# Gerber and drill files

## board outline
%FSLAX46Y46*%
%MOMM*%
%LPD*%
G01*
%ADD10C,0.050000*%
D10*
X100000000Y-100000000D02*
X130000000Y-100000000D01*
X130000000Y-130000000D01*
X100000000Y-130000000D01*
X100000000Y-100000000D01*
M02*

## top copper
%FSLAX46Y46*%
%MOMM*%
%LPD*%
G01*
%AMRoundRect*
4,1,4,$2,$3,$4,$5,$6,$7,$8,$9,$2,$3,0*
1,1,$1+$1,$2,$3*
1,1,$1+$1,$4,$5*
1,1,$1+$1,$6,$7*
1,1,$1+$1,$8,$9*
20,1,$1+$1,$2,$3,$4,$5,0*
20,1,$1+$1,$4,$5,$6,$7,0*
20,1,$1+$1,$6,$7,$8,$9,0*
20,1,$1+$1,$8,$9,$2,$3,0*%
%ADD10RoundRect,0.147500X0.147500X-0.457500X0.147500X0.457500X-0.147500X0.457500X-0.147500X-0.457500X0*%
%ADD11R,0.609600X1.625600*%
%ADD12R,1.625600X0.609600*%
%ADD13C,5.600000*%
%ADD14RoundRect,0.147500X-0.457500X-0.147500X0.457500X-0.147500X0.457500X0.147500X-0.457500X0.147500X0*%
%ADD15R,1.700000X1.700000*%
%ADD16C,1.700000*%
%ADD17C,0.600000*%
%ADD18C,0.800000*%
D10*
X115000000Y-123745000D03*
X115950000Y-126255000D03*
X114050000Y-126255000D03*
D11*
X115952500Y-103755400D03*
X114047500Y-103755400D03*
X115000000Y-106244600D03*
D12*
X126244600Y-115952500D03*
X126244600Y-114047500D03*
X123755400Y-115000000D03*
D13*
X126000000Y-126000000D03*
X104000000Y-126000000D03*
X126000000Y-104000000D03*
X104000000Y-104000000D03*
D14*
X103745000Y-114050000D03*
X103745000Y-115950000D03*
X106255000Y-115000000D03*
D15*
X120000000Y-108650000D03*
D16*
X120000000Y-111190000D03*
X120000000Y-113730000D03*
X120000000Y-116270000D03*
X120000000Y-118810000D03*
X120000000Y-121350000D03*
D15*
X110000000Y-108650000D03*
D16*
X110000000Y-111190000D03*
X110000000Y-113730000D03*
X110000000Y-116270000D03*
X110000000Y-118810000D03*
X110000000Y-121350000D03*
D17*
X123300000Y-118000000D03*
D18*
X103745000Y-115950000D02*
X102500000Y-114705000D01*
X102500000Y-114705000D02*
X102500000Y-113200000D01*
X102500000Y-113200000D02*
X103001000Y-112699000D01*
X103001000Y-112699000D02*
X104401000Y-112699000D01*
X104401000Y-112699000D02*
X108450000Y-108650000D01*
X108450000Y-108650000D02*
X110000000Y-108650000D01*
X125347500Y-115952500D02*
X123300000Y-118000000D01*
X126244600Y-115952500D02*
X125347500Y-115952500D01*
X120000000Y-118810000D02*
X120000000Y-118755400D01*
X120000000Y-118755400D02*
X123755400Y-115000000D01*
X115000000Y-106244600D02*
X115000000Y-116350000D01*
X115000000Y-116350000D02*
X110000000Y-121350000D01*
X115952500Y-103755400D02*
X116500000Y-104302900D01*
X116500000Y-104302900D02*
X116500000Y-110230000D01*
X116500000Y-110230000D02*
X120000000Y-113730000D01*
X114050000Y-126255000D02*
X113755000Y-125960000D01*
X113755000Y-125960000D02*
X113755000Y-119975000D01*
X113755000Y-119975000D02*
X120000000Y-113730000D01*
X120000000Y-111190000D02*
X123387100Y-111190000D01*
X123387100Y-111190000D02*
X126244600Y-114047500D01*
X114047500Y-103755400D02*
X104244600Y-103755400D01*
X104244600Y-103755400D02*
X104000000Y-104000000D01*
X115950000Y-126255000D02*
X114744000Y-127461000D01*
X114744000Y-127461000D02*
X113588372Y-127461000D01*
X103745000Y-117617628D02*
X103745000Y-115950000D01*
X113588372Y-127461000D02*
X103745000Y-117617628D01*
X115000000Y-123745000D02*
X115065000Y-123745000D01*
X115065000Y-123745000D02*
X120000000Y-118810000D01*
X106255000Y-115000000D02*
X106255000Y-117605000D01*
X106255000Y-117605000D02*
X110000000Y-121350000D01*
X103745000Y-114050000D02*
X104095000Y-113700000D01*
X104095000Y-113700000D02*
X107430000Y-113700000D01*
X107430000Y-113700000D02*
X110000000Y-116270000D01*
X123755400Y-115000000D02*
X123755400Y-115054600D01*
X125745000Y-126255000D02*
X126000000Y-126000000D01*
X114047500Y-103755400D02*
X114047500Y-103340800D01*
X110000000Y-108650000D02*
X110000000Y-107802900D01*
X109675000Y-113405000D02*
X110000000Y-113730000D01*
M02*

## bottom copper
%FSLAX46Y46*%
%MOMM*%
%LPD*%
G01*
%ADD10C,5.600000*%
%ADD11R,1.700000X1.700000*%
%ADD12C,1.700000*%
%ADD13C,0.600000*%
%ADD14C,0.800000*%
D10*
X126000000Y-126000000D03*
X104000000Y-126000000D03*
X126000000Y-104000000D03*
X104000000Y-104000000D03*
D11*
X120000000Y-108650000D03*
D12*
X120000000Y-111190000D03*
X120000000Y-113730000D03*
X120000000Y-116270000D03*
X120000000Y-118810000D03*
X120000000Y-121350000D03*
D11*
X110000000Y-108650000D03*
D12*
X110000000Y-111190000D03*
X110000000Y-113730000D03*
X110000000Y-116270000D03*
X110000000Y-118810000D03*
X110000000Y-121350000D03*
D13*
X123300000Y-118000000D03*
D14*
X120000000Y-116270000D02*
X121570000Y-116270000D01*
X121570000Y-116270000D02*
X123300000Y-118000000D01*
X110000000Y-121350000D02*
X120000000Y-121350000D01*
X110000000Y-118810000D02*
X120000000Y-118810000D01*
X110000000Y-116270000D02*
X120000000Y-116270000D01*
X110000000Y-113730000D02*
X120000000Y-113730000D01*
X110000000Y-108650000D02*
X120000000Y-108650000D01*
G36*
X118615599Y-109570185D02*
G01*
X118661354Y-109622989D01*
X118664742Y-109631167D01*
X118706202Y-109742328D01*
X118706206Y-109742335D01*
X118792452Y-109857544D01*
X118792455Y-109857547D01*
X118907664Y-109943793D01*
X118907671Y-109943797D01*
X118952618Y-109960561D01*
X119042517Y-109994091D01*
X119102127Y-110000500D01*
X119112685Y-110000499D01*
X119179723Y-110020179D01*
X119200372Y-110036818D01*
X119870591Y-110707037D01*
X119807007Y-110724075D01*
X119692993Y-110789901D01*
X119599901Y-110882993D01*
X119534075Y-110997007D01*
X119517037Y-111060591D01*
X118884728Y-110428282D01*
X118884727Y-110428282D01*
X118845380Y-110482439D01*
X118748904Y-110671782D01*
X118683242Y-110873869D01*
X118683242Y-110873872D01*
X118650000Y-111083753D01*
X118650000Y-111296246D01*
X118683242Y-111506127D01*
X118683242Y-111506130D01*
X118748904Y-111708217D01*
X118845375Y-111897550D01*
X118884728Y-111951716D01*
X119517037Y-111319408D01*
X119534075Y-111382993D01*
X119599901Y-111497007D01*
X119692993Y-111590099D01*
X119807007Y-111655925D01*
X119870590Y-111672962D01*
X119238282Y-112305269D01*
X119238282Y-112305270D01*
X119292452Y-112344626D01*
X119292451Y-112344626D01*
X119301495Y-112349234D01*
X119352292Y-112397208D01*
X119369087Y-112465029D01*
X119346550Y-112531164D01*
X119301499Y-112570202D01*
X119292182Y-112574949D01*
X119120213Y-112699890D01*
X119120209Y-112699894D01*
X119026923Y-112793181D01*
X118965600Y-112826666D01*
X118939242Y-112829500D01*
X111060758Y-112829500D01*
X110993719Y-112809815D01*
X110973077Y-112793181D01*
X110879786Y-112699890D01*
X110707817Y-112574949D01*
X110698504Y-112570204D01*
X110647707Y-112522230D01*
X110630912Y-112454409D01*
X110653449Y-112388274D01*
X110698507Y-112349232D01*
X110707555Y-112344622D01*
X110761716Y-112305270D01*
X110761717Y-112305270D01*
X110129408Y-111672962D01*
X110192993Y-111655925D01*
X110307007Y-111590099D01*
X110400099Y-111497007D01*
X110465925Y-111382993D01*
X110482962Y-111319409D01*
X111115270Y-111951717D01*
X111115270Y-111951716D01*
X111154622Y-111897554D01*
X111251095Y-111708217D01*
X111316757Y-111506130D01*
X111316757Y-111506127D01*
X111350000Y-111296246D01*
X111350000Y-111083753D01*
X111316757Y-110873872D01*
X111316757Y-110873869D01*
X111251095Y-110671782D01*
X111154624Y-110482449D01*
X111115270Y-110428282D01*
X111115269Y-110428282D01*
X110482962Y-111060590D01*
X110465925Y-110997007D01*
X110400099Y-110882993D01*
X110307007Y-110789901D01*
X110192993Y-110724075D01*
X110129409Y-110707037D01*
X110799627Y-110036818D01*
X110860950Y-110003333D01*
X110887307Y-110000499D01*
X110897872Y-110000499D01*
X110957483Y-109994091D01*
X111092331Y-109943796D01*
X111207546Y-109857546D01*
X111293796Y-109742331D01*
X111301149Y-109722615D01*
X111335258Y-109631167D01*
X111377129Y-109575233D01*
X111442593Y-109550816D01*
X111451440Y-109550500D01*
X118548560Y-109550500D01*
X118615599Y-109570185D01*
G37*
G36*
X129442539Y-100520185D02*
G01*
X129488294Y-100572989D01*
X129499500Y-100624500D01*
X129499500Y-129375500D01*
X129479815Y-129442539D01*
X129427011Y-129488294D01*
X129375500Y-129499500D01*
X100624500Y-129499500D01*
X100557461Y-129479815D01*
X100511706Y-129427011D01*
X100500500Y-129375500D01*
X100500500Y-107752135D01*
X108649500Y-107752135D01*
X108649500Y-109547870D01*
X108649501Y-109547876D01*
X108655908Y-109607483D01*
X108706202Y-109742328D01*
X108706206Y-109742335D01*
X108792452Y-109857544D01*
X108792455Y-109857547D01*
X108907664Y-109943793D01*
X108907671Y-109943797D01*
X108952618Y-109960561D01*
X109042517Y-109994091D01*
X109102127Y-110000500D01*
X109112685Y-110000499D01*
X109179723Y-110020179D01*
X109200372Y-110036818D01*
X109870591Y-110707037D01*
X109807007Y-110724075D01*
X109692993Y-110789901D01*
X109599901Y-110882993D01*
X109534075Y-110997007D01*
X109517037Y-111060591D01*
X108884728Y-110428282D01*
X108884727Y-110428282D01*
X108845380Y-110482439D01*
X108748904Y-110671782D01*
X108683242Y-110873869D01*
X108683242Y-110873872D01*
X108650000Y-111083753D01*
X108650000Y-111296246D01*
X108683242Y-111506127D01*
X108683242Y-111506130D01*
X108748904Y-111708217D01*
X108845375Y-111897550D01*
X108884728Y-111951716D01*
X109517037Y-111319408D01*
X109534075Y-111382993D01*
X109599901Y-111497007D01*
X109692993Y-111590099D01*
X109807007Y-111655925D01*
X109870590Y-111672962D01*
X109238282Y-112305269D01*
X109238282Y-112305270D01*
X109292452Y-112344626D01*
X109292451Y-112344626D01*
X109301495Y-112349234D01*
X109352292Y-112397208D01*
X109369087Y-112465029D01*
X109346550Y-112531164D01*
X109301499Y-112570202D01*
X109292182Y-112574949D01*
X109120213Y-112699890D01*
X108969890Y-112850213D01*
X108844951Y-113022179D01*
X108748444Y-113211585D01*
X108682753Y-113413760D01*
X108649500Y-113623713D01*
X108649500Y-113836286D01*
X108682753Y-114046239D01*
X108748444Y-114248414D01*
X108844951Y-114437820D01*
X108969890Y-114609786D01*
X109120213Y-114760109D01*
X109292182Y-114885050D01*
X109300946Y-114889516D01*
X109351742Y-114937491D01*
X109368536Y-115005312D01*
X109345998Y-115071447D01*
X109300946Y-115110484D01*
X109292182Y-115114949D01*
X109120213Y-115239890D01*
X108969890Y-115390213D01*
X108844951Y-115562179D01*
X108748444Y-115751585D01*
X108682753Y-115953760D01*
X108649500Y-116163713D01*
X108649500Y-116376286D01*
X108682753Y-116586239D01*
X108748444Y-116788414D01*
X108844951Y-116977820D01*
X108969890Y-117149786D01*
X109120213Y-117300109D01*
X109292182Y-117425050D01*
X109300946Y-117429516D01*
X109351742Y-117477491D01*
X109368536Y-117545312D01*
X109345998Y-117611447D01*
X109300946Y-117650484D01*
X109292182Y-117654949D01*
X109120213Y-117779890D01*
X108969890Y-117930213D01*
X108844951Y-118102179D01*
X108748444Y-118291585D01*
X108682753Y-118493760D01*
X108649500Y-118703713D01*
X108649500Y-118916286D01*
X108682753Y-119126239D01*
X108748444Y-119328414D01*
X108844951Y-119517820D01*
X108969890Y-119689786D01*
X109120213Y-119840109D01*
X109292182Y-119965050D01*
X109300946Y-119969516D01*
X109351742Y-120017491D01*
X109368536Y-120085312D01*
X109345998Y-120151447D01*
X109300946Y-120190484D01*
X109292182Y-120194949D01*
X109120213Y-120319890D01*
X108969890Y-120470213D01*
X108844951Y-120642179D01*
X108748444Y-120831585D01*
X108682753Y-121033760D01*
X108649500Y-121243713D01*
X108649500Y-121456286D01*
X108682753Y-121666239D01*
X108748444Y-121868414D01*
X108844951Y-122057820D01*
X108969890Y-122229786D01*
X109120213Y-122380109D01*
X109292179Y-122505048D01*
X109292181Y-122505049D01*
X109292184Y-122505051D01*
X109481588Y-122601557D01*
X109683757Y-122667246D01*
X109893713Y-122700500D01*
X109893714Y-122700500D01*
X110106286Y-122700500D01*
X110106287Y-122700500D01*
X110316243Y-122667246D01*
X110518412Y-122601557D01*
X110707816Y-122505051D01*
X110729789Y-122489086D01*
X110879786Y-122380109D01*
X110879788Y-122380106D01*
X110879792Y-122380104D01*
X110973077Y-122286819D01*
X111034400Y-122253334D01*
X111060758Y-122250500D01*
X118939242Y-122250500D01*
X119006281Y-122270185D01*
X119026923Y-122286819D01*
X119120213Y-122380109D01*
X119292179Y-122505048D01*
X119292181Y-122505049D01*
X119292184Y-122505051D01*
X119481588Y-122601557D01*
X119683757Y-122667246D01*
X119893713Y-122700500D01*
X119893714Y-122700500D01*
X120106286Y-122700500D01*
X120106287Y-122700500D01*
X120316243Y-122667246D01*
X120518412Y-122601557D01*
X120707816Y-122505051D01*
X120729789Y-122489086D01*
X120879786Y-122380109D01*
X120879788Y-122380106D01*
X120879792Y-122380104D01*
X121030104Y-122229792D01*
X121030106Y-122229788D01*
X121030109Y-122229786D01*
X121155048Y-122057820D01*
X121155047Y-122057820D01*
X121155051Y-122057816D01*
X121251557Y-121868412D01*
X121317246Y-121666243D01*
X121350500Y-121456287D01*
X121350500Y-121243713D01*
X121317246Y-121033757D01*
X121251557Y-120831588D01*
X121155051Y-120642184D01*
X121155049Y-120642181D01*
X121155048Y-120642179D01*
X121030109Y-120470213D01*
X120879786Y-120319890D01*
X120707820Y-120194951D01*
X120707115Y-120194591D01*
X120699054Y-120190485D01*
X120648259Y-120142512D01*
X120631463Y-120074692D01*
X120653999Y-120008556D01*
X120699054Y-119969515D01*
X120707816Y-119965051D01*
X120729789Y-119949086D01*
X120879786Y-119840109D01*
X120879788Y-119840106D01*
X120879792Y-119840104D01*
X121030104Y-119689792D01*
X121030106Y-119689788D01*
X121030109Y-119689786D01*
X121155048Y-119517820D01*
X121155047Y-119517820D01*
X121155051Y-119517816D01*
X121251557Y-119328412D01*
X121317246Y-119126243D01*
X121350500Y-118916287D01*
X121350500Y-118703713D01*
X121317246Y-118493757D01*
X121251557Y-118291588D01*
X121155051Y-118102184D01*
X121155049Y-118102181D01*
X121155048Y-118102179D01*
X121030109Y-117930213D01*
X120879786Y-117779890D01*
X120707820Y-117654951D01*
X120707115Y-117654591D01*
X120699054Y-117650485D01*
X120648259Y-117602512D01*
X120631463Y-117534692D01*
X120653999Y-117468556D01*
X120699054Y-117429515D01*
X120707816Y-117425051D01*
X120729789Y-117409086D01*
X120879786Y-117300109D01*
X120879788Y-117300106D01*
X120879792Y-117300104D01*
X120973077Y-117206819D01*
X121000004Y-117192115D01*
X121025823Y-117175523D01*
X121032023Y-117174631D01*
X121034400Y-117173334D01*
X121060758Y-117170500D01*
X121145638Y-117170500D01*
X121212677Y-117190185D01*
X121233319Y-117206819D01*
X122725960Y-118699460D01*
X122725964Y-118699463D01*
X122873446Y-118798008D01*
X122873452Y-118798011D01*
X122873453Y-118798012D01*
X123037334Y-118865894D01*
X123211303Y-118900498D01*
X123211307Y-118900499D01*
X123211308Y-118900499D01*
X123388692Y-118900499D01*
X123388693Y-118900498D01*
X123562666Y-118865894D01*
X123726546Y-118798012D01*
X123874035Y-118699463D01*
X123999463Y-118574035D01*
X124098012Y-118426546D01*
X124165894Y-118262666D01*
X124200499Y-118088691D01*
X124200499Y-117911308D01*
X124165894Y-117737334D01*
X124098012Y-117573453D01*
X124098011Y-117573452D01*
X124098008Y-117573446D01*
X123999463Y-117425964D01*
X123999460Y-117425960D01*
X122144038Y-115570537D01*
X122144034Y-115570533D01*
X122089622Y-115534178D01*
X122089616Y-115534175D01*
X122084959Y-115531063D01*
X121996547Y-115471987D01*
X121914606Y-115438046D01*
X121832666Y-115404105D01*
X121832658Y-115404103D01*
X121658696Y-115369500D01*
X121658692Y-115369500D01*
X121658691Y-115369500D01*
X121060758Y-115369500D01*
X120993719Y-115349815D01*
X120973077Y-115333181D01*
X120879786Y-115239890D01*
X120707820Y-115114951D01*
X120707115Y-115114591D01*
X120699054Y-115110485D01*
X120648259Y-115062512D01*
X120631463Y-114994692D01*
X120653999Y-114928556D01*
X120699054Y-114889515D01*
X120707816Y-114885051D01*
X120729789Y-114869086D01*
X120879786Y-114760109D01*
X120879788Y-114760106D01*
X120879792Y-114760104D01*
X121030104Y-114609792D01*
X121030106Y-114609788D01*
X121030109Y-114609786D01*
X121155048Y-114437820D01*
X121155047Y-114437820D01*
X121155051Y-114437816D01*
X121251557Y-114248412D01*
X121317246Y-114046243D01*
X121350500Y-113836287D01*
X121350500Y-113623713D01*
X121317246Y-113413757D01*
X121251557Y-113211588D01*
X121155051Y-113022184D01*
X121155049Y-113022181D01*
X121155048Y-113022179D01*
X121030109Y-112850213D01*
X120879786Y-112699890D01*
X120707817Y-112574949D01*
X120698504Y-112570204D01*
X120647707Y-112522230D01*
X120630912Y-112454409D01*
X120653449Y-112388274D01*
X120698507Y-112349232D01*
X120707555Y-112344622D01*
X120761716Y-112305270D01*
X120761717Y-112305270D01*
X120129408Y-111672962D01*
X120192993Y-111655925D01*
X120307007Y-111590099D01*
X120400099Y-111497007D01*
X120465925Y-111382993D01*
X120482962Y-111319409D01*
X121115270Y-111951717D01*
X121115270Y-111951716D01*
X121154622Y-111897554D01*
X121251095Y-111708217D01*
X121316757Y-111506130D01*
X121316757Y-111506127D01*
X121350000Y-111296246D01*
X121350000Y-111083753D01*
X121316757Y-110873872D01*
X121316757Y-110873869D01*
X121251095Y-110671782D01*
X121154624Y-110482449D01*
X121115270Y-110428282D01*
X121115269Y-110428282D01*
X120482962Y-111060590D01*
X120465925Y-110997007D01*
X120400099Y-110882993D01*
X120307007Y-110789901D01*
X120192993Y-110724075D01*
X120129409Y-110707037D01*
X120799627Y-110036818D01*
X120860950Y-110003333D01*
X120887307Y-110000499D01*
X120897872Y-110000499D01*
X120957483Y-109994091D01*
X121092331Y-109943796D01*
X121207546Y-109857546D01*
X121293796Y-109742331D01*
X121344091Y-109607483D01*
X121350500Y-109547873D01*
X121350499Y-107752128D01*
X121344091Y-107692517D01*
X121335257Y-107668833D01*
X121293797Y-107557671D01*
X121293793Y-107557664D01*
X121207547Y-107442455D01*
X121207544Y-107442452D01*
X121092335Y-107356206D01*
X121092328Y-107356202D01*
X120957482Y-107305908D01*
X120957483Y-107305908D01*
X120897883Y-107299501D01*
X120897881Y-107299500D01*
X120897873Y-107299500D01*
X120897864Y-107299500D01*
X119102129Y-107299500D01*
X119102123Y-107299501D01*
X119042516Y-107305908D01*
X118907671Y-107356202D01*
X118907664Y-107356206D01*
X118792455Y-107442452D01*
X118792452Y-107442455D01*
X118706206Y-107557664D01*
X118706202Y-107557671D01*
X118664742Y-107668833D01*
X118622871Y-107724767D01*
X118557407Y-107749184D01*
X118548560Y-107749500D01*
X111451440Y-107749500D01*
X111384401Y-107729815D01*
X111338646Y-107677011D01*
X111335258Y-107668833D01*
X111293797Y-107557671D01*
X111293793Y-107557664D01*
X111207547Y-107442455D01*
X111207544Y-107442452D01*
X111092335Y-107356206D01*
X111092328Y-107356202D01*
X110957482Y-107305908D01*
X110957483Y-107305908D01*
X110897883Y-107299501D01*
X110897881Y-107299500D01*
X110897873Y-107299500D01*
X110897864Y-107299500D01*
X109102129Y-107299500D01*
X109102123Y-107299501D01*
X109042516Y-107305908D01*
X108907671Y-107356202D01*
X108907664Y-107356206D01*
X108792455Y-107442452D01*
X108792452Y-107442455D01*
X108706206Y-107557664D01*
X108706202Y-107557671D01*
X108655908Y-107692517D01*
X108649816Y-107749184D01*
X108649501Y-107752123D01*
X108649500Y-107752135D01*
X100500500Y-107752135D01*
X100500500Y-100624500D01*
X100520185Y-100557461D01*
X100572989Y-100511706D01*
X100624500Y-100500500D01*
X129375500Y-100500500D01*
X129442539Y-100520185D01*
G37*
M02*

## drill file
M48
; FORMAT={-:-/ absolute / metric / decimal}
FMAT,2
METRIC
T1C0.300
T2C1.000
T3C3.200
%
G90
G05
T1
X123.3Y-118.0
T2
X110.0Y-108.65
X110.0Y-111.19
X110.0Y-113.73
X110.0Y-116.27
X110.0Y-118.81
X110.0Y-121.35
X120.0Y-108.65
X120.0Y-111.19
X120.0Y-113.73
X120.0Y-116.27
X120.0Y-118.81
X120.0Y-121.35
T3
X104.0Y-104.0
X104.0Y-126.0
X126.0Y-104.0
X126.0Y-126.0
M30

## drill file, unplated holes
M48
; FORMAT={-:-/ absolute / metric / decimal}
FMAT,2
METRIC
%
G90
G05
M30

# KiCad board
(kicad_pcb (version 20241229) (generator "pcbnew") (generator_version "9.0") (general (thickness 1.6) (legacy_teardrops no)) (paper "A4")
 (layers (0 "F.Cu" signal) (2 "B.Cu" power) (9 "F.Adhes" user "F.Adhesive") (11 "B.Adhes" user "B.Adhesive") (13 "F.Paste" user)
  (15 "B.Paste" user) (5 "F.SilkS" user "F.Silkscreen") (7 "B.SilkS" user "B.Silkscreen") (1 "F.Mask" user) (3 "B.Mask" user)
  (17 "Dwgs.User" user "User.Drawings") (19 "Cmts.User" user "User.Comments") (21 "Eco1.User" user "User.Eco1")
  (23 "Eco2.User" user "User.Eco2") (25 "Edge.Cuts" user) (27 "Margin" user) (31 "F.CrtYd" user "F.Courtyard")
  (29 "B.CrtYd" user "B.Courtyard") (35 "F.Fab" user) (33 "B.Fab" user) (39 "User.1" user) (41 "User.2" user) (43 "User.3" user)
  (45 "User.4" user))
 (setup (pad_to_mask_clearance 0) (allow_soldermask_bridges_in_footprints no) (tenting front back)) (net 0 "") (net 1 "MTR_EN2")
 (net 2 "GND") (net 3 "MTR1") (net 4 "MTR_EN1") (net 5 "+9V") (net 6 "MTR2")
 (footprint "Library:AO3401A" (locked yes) (layer "F.Cu") (at 125 115 90)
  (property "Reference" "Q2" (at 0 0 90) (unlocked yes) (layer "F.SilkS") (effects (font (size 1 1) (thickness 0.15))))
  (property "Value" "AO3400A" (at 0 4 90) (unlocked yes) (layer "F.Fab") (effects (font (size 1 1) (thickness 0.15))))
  (pad "1" smd rect (at -0.9525 1.2446 90) (size 0.6096 1.6256) (layers "F.Cu" "F.Mask" "F.Paste") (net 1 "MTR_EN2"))
  (pad "2" smd rect (at 0.9525 1.2446 90) (size 0.6096 1.6256) (layers "F.Cu" "F.Mask" "F.Paste") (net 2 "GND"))
  (pad "3" smd rect (at 0 -1.2446 90) (size 0.6096 1.6256) (layers "F.Cu" "F.Mask" "F.Paste") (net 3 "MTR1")))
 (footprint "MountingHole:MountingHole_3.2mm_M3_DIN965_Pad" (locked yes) (layer "F.Cu") (at 104 104)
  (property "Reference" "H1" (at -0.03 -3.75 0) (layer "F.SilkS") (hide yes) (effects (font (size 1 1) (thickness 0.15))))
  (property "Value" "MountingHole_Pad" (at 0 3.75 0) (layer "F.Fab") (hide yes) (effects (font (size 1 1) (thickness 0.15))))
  (pad "1" thru_hole circle (at 0 0) (size 5.6 5.6) (drill 3.2) (layers "*.Cu" "*.Mask") (remove_unused_layers no) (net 2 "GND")
   (zone_connect 2)))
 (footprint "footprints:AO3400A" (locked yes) (layer "F.Cu") (at 115 125 90)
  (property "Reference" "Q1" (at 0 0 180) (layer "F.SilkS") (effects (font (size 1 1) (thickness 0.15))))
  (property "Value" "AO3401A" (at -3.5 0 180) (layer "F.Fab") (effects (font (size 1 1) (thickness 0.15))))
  (pad "1" smd roundrect (at -1.255 -0.95 90) (size 1.21 0.59) (layers "F.Cu" "F.Mask" "F.Paste") (roundrect_rratio 0.25) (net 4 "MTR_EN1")
   (solder_mask_margin 0.102))
  (pad "2" smd roundrect (at -1.255 0.95 90) (size 1.21 0.59) (layers "F.Cu" "F.Mask" "F.Paste") (roundrect_rratio 0.25) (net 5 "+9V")
   (solder_mask_margin 0.102))
  (pad "3" smd roundrect (at 1.255 0 90) (size 1.21 0.59) (layers "F.Cu" "F.Mask" "F.Paste") (roundrect_rratio 0.25) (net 3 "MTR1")
   (solder_mask_margin 0.102)))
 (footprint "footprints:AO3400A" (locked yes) (layer "F.Cu") (at 105 115)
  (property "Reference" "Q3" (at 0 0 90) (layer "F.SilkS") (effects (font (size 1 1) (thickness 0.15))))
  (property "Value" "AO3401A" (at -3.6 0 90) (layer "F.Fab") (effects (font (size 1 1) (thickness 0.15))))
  (pad "1" smd roundrect (at -1.255 -0.95) (size 1.21 0.59) (layers "F.Cu" "F.Mask" "F.Paste") (roundrect_rratio 0.25) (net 1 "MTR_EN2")
   (solder_mask_margin 0.102))
  (pad "2" smd roundrect (at -1.255 0.95) (size 1.21 0.59) (layers "F.Cu" "F.Mask" "F.Paste") (roundrect_rratio 0.25) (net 5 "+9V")
   (solder_mask_margin 0.102))
  (pad "3" smd roundrect (at 1.255 0) (size 1.21 0.59) (layers "F.Cu" "F.Mask" "F.Paste") (roundrect_rratio 0.25) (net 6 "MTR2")
   (solder_mask_margin 0.102)))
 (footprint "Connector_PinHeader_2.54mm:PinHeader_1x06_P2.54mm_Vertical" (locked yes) (layer "F.Cu") (at 120 108.65)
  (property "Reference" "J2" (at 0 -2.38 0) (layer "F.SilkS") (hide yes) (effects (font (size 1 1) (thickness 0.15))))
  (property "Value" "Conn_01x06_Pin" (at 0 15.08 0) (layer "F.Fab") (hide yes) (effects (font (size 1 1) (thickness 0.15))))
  (pad "1" thru_hole rect (at 0 0) (size 1.7 1.7) (drill 1) (layers "*.Cu" "*.Mask") (remove_unused_layers no) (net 5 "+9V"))
  (pad "2" thru_hole circle (at 0 2.54) (size 1.7 1.7) (drill 1) (layers "*.Cu" "*.Mask") (remove_unused_layers no) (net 2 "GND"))
  (pad "3" thru_hole circle (at 0 5.08) (size 1.7 1.7) (drill 1) (layers "*.Cu" "*.Mask") (remove_unused_layers no) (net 4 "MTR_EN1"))
  (pad "4" thru_hole circle (at 0 7.62) (size 1.7 1.7) (drill 1) (layers "*.Cu" "*.Mask") (remove_unused_layers no) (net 1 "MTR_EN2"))
  (pad "5" thru_hole circle (at 0 10.16) (size 1.7 1.7) (drill 1) (layers "*.Cu" "*.Mask") (remove_unused_layers no) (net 3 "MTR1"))
  (pad "6" thru_hole circle (at 0 12.7) (size 1.7 1.7) (drill 1) (layers "*.Cu" "*.Mask") (remove_unused_layers no) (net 6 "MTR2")))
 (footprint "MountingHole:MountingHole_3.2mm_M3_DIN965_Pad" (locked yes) (layer "F.Cu") (at 104 126)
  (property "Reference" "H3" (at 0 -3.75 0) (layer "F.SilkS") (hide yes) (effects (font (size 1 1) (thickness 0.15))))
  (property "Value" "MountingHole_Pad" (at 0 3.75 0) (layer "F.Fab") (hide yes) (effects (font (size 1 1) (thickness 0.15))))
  (pad "1" thru_hole circle (at 0 0) (size 5.6 5.6) (drill 3.2) (layers "*.Cu" "*.Mask") (remove_unused_layers no) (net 2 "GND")
   (zone_connect 2)))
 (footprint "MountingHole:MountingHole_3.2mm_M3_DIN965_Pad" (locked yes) (layer "F.Cu") (at 126 126)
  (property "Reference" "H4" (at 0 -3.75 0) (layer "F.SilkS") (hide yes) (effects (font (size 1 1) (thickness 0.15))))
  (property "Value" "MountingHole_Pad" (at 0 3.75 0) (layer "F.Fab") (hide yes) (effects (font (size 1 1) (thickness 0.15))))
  (pad "1" thru_hole circle (at 0 0) (size 5.6 5.6) (drill 3.2) (layers "*.Cu" "*.Mask") (remove_unused_layers no) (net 2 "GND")
   (zone_connect 2)))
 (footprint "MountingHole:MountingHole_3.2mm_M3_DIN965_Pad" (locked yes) (layer "F.Cu") (at 126 104)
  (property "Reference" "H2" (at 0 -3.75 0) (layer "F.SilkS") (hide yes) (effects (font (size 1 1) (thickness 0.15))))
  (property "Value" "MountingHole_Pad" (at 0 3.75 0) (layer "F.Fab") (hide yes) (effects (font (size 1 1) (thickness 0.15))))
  (pad "1" thru_hole circle (at 0 0) (size 5.6 5.6) (drill 3.2) (layers "*.Cu" "*.Mask") (remove_unused_layers no) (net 2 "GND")
   (zone_connect 2)))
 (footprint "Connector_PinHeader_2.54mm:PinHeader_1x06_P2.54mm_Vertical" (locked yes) (layer "F.Cu") (at 110 108.65)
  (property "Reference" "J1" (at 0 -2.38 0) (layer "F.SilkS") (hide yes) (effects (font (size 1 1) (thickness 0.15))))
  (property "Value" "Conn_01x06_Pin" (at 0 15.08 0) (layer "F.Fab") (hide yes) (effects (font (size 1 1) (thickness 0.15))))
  (pad "1" thru_hole rect (at 0 0) (size 1.7 1.7) (drill 1) (layers "*.Cu" "*.Mask") (remove_unused_layers no) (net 5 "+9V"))
  (pad "2" thru_hole circle (at 0 2.54) (size 1.7 1.7) (drill 1) (layers "*.Cu" "*.Mask") (remove_unused_layers no) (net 2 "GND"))
  (pad "3" thru_hole circle (at 0 5.08) (size 1.7 1.7) (drill 1) (layers "*.Cu" "*.Mask") (remove_unused_layers no) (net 4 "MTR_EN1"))
  (pad "4" thru_hole circle (at 0 7.62) (size 1.7 1.7) (drill 1) (layers "*.Cu" "*.Mask") (remove_unused_layers no) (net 1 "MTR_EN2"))
  (pad "5" thru_hole circle (at 0 10.16) (size 1.7 1.7) (drill 1) (layers "*.Cu" "*.Mask") (remove_unused_layers no) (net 3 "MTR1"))
  (pad "6" thru_hole circle (at 0 12.7) (size 1.7 1.7) (drill 1) (layers "*.Cu" "*.Mask") (remove_unused_layers no) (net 6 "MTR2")))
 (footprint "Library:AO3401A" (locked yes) (layer "F.Cu") (at 115 105 180)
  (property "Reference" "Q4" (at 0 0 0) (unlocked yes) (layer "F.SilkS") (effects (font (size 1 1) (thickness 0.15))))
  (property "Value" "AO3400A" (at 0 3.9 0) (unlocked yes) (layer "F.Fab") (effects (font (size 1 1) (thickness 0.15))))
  (pad "1" smd rect (at -0.9525 1.2446 180) (size 0.6096 1.6256) (layers "F.Cu" "F.Mask" "F.Paste") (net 4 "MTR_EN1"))
  (pad "2" smd rect (at 0.9525 1.2446 180) (size 0.6096 1.6256) (layers "F.Cu" "F.Mask" "F.Paste") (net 2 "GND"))
  (pad "3" smd rect (at 0 -1.2446 180) (size 0.6096 1.6256) (layers "F.Cu" "F.Mask" "F.Paste") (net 6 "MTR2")))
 (gr_rect (start 100 100) (end 130 130) (stroke (width 0.05) (type default)) (fill no) (layer "Edge.Cuts"))
 (segment (start 103.745 117.617628) (end 103.745 115.95) (width 0.8) (layer "F.Cu") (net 5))
 (segment (start 104.401 112.699) (end 108.45 108.65) (width 0.8) (layer "F.Cu") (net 5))
 (segment (start 102.5 113.2) (end 103.001 112.699) (width 0.8) (layer "F.Cu") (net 5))
 (segment (start 102.5 114.705) (end 102.5 113.2) (width 0.8) (layer "F.Cu") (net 5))
 (segment (start 103.001 112.699) (end 104.401 112.699) (width 0.8) (layer "F.Cu") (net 5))
 (segment (start 114.744 127.461) (end 113.588372 127.461) (width 0.8) (layer "F.Cu") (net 5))
 (segment (start 113.588372 127.461) (end 103.745 117.617628) (width 0.8) (layer "F.Cu") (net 5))
 (segment (start 110 108.65) (end 110 107.8029) (width 0.8) (layer "F.Cu") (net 5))
 (segment (start 115.95 126.255) (end 114.744 127.461) (width 0.8) (layer "F.Cu") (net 5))
 (segment (start 108.45 108.65) (end 110 108.65) (width 0.8) (layer "F.Cu") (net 5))
 (segment (start 103.745 115.95) (end 102.5 114.705) (width 0.8) (layer "F.Cu") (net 5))
 (segment (start 110 108.65) (end 120 108.65) (width 0.8) (layer "B.Cu") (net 5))
 (segment (start 115.9525 103.7554) (end 116.5 104.3029) (width 0.8) (layer "F.Cu") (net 4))
 (segment (start 109.675 113.405) (end 110 113.73) (width 0.8) (layer "F.Cu") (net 4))
 (segment (start 113.755 125.96) (end 113.755 119.975) (width 0.8) (layer "F.Cu") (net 4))
 (segment (start 116.5 110.23) (end 120 113.73) (width 0.8) (layer "F.Cu") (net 4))
 (segment (start 113.755 119.975) (end 120 113.73) (width 0.8) (layer "F.Cu") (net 4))
 (segment (start 114.05 126.255) (end 113.755 125.96) (width 0.8) (layer "F.Cu") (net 4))
 (segment (start 116.5 104.3029) (end 116.5 110.23) (width 0.8) (layer "F.Cu") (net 4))
 (segment (start 110 113.73) (end 120 113.73) (width 0.8) (layer "B.Cu") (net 4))
 (segment (start 120 111.19) (end 123.3871 111.19) (width 0.8) (layer "F.Cu") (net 2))
 (segment (start 114.0475 103.7554) (end 114.0475 103.3408) (width 0.8) (layer "F.Cu") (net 2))
 (segment (start 125.745 126.255) (end 126 126) (width 0.8) (layer "F.Cu") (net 2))
 (segment (start 114.0475 103.7554) (end 104.2446 103.7554) (width 0.8) (layer "F.Cu") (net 2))
 (segment (start 123.3871 111.19) (end 126.2446 114.0475) (width 0.8) (layer "F.Cu") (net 2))
 (segment (start 104.2446 103.7554) (end 104 104) (width 0.8) (layer "F.Cu") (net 2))
 (segment (start 115 116.35) (end 110 121.35) (width 0.8) (layer "F.Cu") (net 6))
 (segment (start 115 106.2446) (end 115 116.35) (width 0.8) (layer "F.Cu") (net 6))
 (segment (start 106.255 115) (end 106.255 117.605) (width 0.8) (layer "F.Cu") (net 6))
 (segment (start 106.255 117.605) (end 110 121.35) (width 0.8) (layer "F.Cu") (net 6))
 (segment (start 110 121.35) (end 120 121.35) (width 0.8) (layer "B.Cu") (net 6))
 (segment (start 120 118.7554) (end 123.7554 115) (width 0.8) (layer "F.Cu") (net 3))
 (segment (start 115 123.745) (end 115.065 123.745) (width 0.8) (layer "F.Cu") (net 3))
 (segment (start 120 118.81) (end 120 118.7554) (width 0.8) (layer "F.Cu") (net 3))
 (segment (start 123.7554 115) (end 123.7554 115.0546) (width 0.8) (layer "F.Cu") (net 3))
 (segment (start 115.065 123.745) (end 120 118.81) (width 0.8) (layer "F.Cu") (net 3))
 (segment (start 110 118.81) (end 120 118.81) (width 0.8) (layer "B.Cu") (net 3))
 (segment (start 125.3475 115.9525) (end 123.3 118) (width 0.8) (layer "F.Cu") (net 1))
 (segment (start 103.745 114.05) (end 104.095 113.7) (width 0.8) (layer "F.Cu") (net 1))
 (segment (start 126.2446 115.9525) (end 125.3475 115.9525) (width 0.8) (layer "F.Cu") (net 1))
 (segment (start 104.095 113.7) (end 107.43 113.7) (width 0.8) (layer "F.Cu") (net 1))
 (segment (start 107.43 113.7) (end 110 116.27) (width 0.8) (layer "F.Cu") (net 1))
 (via (at 123.3 118) (size 0.6) (drill 0.3) (layers "F.Cu" "B.Cu") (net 1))
 (segment (start 120 116.27) (end 121.57 116.27) (width 0.8) (layer "B.Cu") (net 1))
 (segment (start 110 116.27) (end 120 116.27) (width 0.8) (layer "B.Cu") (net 1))
 (segment (start 121.57 116.27) (end 123.3 118) (width 0.8) (layer "B.Cu") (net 1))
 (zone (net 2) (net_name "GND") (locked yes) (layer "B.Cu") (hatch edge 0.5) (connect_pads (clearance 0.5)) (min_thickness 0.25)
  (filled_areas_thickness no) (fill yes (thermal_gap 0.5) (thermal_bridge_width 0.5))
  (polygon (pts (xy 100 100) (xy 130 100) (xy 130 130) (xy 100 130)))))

